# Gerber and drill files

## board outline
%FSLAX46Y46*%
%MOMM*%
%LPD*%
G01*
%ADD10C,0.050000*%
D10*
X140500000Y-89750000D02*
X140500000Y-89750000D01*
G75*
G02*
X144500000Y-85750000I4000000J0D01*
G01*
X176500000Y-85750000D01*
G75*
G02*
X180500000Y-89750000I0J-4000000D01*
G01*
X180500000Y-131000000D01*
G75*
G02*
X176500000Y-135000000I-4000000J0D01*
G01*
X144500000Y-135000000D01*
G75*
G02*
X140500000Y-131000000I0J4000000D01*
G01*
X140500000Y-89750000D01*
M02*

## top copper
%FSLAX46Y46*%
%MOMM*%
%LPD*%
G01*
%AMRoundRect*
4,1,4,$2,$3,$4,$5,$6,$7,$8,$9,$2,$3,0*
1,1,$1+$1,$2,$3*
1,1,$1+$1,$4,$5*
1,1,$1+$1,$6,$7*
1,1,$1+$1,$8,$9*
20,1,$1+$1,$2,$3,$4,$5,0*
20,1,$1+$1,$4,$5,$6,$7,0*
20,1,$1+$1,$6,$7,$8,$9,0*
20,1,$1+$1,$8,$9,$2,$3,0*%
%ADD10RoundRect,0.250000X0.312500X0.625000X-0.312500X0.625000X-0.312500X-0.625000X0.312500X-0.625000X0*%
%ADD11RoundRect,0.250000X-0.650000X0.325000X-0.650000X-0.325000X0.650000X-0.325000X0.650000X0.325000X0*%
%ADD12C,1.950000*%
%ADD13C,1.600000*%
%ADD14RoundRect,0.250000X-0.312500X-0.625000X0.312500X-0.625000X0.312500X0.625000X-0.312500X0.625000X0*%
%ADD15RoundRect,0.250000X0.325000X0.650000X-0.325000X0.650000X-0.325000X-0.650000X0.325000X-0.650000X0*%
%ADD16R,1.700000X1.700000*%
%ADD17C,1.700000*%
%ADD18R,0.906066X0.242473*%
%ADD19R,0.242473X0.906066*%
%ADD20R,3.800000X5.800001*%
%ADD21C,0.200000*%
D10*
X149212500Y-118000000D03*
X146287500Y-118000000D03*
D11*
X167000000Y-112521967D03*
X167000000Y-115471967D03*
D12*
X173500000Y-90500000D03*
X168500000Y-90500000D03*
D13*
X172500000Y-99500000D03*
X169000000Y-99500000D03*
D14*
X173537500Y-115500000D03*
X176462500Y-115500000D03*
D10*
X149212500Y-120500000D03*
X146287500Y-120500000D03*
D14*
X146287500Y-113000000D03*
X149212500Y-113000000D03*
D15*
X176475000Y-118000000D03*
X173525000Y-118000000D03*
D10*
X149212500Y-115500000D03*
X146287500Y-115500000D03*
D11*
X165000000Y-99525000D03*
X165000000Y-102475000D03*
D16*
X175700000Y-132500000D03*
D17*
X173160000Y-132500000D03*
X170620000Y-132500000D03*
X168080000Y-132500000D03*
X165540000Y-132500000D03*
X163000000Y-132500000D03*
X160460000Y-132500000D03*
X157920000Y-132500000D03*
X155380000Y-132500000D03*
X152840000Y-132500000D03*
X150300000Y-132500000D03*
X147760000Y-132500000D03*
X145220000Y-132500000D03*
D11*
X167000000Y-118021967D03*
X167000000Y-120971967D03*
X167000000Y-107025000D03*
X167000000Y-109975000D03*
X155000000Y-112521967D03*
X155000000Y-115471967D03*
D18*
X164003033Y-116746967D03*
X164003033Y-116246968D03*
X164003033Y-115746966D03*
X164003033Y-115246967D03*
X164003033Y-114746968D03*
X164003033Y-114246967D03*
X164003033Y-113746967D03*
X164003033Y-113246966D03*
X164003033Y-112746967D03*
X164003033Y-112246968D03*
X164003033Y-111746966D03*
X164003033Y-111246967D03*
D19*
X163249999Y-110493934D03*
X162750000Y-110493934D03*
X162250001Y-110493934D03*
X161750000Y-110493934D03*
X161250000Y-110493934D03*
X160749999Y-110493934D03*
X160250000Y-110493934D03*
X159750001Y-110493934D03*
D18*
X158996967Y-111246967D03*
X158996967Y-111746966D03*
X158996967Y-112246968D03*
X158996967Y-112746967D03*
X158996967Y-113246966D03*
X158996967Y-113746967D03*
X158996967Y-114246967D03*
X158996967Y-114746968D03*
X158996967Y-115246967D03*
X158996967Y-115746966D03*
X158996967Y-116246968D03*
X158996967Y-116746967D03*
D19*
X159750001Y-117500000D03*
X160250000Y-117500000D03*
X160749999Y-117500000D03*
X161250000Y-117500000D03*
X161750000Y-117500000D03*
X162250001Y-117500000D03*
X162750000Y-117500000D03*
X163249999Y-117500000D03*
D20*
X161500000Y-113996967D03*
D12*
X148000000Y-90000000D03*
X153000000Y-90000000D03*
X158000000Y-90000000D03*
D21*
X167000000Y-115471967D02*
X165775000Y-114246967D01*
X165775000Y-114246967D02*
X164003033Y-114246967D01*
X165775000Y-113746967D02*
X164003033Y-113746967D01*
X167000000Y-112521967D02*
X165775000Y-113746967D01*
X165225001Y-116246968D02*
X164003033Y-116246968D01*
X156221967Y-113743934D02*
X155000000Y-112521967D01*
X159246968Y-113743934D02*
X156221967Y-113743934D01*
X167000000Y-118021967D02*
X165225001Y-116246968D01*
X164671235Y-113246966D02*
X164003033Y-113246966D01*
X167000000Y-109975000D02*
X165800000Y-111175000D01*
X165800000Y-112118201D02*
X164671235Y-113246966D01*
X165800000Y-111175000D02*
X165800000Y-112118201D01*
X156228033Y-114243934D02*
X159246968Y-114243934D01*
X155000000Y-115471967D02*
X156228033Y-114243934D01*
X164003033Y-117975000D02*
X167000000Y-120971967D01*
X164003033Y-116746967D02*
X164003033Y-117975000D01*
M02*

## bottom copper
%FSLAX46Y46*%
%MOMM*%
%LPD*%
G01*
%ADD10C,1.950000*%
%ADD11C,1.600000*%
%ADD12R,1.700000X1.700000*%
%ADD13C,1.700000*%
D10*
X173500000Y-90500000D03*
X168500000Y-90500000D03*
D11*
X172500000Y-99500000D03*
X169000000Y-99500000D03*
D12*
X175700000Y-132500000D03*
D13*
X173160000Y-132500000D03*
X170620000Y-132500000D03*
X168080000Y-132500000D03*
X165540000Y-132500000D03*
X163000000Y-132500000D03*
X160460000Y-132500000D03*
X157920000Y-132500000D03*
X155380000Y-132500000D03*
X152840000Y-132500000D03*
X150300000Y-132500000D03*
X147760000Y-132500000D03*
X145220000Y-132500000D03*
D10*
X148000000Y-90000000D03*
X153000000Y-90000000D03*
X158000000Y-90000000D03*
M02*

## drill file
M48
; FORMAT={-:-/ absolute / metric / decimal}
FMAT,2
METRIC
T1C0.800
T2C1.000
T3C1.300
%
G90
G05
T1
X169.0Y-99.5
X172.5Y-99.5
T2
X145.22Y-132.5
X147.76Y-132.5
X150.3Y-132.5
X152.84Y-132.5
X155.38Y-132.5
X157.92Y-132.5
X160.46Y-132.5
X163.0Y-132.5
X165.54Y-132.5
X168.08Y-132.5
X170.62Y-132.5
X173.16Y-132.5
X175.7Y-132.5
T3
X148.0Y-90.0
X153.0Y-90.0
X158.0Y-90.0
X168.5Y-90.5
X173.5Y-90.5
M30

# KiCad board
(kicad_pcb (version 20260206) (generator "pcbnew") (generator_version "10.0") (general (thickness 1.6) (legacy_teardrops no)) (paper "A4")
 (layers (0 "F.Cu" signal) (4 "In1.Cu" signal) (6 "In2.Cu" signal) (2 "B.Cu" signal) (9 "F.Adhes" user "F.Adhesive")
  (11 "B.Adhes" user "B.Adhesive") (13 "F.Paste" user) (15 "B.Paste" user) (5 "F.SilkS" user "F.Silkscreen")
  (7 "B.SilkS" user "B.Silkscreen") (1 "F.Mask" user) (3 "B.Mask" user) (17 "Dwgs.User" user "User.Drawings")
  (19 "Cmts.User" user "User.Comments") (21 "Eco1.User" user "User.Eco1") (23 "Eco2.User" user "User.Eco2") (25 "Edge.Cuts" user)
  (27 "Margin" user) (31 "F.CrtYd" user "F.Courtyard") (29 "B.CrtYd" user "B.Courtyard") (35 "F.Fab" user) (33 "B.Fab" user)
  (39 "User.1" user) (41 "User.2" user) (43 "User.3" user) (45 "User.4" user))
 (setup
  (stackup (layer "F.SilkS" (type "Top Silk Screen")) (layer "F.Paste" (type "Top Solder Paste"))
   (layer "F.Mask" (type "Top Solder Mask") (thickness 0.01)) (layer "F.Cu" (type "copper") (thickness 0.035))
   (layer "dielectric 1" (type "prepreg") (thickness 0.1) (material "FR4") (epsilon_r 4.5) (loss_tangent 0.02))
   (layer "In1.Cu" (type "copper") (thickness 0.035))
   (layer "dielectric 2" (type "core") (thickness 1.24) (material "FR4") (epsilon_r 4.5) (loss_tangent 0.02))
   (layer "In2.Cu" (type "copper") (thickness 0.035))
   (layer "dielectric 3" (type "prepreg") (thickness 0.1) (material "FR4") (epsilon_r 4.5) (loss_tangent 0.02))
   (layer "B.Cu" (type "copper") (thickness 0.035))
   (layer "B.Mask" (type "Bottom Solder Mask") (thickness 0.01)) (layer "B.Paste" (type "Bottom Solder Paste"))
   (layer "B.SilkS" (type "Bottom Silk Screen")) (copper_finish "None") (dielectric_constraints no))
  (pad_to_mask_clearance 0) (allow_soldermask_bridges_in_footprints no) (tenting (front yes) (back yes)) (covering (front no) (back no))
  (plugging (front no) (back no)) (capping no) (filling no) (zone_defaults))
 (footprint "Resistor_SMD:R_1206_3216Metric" (layer "F.Cu") (at 147.75 118 180)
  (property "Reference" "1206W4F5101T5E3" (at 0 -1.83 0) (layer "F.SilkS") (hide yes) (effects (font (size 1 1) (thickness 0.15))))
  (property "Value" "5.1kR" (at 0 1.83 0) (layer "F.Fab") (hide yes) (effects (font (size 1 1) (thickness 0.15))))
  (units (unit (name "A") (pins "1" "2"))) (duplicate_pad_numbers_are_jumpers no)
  (pad "1" smd roundrect (at -1.4625 0 180) (size 1.125 1.75) (layers "F.Cu" "F.Mask" "F.Paste") (roundrect_rratio 0.222222)
   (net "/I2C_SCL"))
  (pad "2" smd roundrect (at 1.4625 0 180) (size 1.125 1.75) (layers "F.Cu" "F.Mask" "F.Paste") (roundrect_rratio 0.222222) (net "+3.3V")))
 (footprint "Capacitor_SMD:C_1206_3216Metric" (layer "F.Cu") (at 167 113.996967 -90)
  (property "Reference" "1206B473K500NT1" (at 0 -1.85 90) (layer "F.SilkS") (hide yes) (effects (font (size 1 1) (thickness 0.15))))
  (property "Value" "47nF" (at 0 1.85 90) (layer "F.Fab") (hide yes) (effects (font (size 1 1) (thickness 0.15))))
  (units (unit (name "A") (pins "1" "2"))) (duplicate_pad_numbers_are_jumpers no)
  (pad "1" smd roundrect (at -1.475 0 270) (size 1.15 1.8) (layers "F.Cu" "F.Mask" "F.Paste") (roundrect_rratio 0.217391) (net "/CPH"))
  (pad "2" smd roundrect (at 1.475 0 270) (size 1.15 1.8) (layers "F.Cu" "F.Mask" "F.Paste") (roundrect_rratio 0.217391) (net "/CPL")))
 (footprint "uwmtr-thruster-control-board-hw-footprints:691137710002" (layer "F.Cu") (at 171 90.5 180)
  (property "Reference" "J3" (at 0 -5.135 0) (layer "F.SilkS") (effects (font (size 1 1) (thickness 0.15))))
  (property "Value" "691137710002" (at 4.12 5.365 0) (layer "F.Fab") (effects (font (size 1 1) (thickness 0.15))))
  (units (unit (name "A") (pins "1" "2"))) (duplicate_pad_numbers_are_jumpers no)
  (pad "1" thru_hole circle (at -2.5 0 180) (size 1.95 1.95) (drill 1.3) (layers "*.Cu" "*.Mask") (remove_unused_layers no) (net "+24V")
   (solder_mask_margin 0.102))
  (pad "2" thru_hole circle (at 2.5 0 180) (size 1.95 1.95) (drill 1.3) (layers "*.Cu" "*.Mask") (remove_unused_layers no) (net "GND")
   (solder_mask_margin 0.102)))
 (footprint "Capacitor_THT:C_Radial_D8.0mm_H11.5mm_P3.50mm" (layer "F.Cu") (at 172.5 99.5 180)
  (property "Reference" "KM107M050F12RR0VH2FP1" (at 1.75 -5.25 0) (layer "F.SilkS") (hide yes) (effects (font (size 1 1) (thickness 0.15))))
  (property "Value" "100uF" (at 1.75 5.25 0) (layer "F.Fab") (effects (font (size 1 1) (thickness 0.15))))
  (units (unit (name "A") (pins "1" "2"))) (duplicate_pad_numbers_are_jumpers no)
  (pad "1" thru_hole circle (at 0 0 180) (size 1.6 1.6) (drill 0.8) (layers "*.Cu" "*.Mask") (remove_unused_layers no) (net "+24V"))
  (pad "2" thru_hole circle (at 3.5 0 180) (size 1.6 1.6) (drill 0.8) (layers "*.Cu" "*.Mask") (remove_unused_layers no) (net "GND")))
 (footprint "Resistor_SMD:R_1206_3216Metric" (layer "F.Cu") (at 175 115.5)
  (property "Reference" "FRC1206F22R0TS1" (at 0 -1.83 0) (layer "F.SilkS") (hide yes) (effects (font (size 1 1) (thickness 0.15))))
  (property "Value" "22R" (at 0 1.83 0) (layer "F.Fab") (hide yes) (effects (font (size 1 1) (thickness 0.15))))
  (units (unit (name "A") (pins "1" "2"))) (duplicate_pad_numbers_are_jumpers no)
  (pad "1" smd roundrect (at -1.4625 0) (size 1.125 1.75) (layers "F.Cu" "F.Mask" "F.Paste") (roundrect_rratio 0.222222) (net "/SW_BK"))
  (pad "2" smd roundrect (at 1.4625 0) (size 1.125 1.75) (layers "F.Cu" "F.Mask" "F.Paste") (roundrect_rratio 0.222222) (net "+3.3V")))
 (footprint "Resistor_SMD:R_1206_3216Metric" (layer "F.Cu") (at 147.75 120.5 180)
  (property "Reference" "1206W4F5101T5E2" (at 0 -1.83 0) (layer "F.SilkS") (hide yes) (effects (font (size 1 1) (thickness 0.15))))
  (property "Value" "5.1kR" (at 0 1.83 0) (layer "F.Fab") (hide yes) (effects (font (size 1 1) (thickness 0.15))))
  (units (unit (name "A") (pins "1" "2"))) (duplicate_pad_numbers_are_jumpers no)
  (pad "1" smd roundrect (at -1.4625 0 180) (size 1.125 1.75) (layers "F.Cu" "F.Mask" "F.Paste") (roundrect_rratio 0.222222)
   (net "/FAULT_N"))
  (pad "2" smd roundrect (at 1.4625 0 180) (size 1.125 1.75) (layers "F.Cu" "F.Mask" "F.Paste") (roundrect_rratio 0.222222) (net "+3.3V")))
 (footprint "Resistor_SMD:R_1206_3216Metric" (layer "F.Cu") (at 147.75 113)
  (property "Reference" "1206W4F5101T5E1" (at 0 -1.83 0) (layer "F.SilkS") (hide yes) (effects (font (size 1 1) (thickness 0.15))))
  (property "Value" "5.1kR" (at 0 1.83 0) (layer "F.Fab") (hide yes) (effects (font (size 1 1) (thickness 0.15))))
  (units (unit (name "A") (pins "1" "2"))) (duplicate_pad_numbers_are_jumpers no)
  (pad "1" smd roundrect (at -1.4625 0) (size 1.125 1.75) (layers "F.Cu" "F.Mask" "F.Paste") (roundrect_rratio 0.222222) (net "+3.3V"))
  (pad "2" smd roundrect (at 1.4625 0) (size 1.125 1.75) (layers "F.Cu" "F.Mask" "F.Paste") (roundrect_rratio 0.222222) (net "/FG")))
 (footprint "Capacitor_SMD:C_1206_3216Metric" (layer "F.Cu") (at 175 118 180)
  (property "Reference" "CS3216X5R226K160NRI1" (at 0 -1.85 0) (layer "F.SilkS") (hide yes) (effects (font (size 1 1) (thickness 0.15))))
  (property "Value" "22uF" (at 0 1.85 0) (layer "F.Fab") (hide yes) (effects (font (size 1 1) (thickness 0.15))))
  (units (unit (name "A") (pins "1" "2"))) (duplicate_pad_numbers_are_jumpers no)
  (pad "1" smd roundrect (at -1.475 0 180) (size 1.15 1.8) (layers "F.Cu" "F.Mask" "F.Paste") (roundrect_rratio 0.217391) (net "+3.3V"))
  (pad "2" smd roundrect (at 1.475 0 180) (size 1.15 1.8) (layers "F.Cu" "F.Mask" "F.Paste") (roundrect_rratio 0.217391) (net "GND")))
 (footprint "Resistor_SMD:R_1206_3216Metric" (layer "F.Cu") (at 147.75 115.5 180)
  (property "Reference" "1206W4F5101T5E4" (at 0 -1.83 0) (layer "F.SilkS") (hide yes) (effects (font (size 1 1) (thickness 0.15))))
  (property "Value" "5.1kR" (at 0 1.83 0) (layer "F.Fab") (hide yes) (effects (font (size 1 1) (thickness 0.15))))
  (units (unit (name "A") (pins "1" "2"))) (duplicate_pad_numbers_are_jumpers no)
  (pad "1" smd roundrect (at -1.4625 0 180) (size 1.125 1.75) (layers "F.Cu" "F.Mask" "F.Paste") (roundrect_rratio 0.222222)
   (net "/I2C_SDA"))
  (pad "2" smd roundrect (at 1.4625 0 180) (size 1.125 1.75) (layers "F.Cu" "F.Mask" "F.Paste") (roundrect_rratio 0.222222) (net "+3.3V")))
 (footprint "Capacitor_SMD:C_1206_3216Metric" (layer "F.Cu") (at 165 101 -90)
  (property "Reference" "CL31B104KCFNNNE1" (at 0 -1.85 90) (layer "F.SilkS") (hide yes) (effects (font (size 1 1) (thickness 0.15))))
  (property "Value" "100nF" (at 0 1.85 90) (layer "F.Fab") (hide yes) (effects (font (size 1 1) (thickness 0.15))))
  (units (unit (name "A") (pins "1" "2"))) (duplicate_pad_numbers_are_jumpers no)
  (pad "1" smd roundrect (at -1.475 0 270) (size 1.15 1.8) (layers "F.Cu" "F.Mask" "F.Paste") (roundrect_rratio 0.217391) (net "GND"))
  (pad "2" smd roundrect (at 1.475 0 270) (size 1.15 1.8) (layers "F.Cu" "F.Mask" "F.Paste") (roundrect_rratio 0.217391) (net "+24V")))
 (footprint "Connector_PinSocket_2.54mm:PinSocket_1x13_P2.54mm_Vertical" (layer "F.Cu") (at 175.7 132.5 -90)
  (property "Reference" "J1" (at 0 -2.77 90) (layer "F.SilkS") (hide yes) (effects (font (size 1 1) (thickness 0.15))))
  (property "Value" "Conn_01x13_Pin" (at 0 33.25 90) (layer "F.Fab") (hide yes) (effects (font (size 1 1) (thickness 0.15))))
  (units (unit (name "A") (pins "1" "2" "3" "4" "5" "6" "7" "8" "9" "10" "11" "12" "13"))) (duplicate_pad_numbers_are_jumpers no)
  (pad "1" thru_hole rect (at 0 0 270) (size 1.7 1.7) (drill 1) (layers "*.Cu" "*.Mask") (remove_unused_layers no) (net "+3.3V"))
  (pad "2" thru_hole circle (at 0 2.54 270) (size 1.7 1.7) (drill 1) (layers "*.Cu" "*.Mask") (remove_unused_layers no) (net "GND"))
  (pad "3" thru_hole circle (at 0 5.08 270) (size 1.7 1.7) (drill 1) (layers "*.Cu" "*.Mask") (remove_unused_layers no) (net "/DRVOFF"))
  (pad "4" thru_hole circle (at 0 7.62 270) (size 1.7 1.7) (drill 1) (layers "*.Cu" "*.Mask") (remove_unused_layers no) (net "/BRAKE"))
  (pad "5" thru_hole circle (at 0 10.16 270) (size 1.7 1.7) (drill 1) (layers "*.Cu" "*.Mask") (remove_unused_layers no) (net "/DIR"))
  (pad "6" thru_hole circle (at 0 12.7 270) (size 1.7 1.7) (drill 1) (layers "*.Cu" "*.Mask") (remove_unused_layers no) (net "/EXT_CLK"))
  (pad "7" thru_hole circle (at 0 15.24 270) (size 1.7 1.7) (drill 1) (layers "*.Cu" "*.Mask") (remove_unused_layers no) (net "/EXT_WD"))
  (pad "8" thru_hole circle (at 0 17.78 270) (size 1.7 1.7) (drill 1) (layers "*.Cu" "*.Mask") (remove_unused_layers no) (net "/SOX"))
  (pad "9" thru_hole circle (at 0 20.32 270) (size 1.7 1.7) (drill 1) (layers "*.Cu" "*.Mask") (remove_unused_layers no) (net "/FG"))
  (pad "10" thru_hole circle (at 0 22.86 270) (size 1.7 1.7) (drill 1) (layers "*.Cu" "*.Mask") (remove_unused_layers no) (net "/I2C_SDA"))
  (pad "11" thru_hole circle (at 0 25.4 270) (size 1.7 1.7) (drill 1) (layers "*.Cu" "*.Mask") (remove_unused_layers no) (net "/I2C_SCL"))
  (pad "12" thru_hole circle (at 0 27.94 270) (size 1.7 1.7) (drill 1) (layers "*.Cu" "*.Mask") (remove_unused_layers no) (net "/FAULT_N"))
  (pad "13" thru_hole circle (at 0 30.48 270) (size 1.7 1.7) (drill 1) (layers "*.Cu" "*.Mask") (remove_unused_layers no)
   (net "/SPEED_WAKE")))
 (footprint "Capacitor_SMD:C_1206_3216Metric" (layer "F.Cu") (at 167 119.496967 -90)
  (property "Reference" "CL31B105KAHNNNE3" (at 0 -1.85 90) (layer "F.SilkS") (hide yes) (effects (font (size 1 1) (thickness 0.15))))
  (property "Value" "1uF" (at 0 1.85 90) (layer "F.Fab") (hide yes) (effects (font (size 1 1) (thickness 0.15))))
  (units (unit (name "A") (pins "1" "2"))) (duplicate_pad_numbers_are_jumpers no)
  (pad "1" smd roundrect (at -1.475 0 270) (size 1.15 1.8) (layers "F.Cu" "F.Mask" "F.Paste") (roundrect_rratio 0.217391) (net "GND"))
  (pad "2" smd roundrect (at 1.475 0 270) (size 1.15 1.8) (layers "F.Cu" "F.Mask" "F.Paste") (roundrect_rratio 0.217391) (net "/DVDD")))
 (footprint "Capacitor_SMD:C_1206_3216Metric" (layer "F.Cu") (at 167 108.5 -90)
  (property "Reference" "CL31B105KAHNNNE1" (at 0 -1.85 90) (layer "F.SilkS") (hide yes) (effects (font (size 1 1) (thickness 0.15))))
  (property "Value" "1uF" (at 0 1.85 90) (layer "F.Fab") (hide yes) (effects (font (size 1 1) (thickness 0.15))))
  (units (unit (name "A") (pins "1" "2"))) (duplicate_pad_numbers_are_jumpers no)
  (pad "1" smd roundrect (at -1.475 0 270) (size 1.15 1.8) (layers "F.Cu" "F.Mask" "F.Paste") (roundrect_rratio 0.217391) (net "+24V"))
  (pad "2" smd roundrect (at 1.475 0 270) (size 1.15 1.8) (layers "F.Cu" "F.Mask" "F.Paste") (roundrect_rratio 0.217391) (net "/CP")))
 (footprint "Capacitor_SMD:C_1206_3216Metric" (layer "F.Cu") (at 155 113.996967 -90)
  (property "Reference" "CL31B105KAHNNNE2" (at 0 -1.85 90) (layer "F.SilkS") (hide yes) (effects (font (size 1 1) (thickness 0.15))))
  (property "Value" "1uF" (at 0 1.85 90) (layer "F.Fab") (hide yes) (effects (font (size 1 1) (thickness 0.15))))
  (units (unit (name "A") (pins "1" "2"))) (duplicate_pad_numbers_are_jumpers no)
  (pad "1" smd roundrect (at -1.475 0 270) (size 1.15 1.8) (layers "F.Cu" "F.Mask" "F.Paste") (roundrect_rratio 0.217391) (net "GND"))
  (pad "2" smd roundrect (at 1.475 0 270) (size 1.15 1.8) (layers "F.Cu" "F.Mask" "F.Paste") (roundrect_rratio 0.217391) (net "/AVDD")))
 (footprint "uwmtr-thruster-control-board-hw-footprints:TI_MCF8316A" (layer "F.Cu") (at 161.5 113.996967 180)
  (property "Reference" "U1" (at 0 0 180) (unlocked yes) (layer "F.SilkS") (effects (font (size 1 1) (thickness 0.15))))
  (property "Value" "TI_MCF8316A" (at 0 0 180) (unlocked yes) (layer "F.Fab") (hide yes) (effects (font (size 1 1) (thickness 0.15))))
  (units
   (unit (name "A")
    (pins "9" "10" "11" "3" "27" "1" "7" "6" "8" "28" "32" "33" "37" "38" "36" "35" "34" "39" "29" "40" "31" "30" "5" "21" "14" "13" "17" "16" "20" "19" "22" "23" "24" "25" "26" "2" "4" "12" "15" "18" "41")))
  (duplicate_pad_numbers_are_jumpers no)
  (pad "1" smd rect (at -2.503033 -2.75 270) (size 0.242473 0.906066) (layers "F.Cu" "F.Mask" "F.Paste") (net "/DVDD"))
  (pad "2" smd rect (at -2.503033 -2.250001 270) (size 0.242473 0.906066) (layers "F.Cu" "F.Mask" "F.Paste") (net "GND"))
  (pad "3" smd rect (at -2.503033 -1.749999 270) (size 0.242473 0.906066) (layers "F.Cu" "F.Mask" "F.Paste") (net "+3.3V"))
  (pad "4" smd rect (at -2.503033 -1.25 270) (size 0.242473 0.906066) (layers "F.Cu" "F.Mask" "F.Paste") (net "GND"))
  (pad "5" smd rect (at -2.503033 -0.750001 270) (size 0.242473 0.906066) (layers "F.Cu" "F.Mask" "F.Paste") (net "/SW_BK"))
  (pad "6" smd rect (at -2.503033 -0.25 270) (size 0.242473 0.906066) (layers "F.Cu" "F.Mask" "F.Paste") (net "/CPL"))
  (pad "7" smd rect (at -2.503033 0.25 270) (size 0.242473 0.906066) (layers "F.Cu" "F.Mask" "F.Paste") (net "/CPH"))
  (pad "8" smd rect (at -2.503033 0.750001 270) (size 0.242473 0.906066) (layers "F.Cu" "F.Mask" "F.Paste") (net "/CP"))
  (pad "9" smd rect (at -2.503033 1.25 270) (size 0.242473 0.906066) (layers "F.Cu" "F.Mask" "F.Paste") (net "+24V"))
  (pad "10" smd rect (at -2.503033 1.749999 270) (size 0.242473 0.906066) (layers "F.Cu" "F.Mask" "F.Paste") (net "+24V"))
  (pad "11" smd rect (at -2.503033 2.250001 270) (size 0.242473 0.906066) (layers "F.Cu" "F.Mask" "F.Paste") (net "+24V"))
  (pad "12" smd rect (at -2.503033 2.75 270) (size 0.242473 0.906066) (layers "F.Cu" "F.Mask" "F.Paste") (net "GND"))
  (pad "13" smd rect (at -1.749999 3.503033 180) (size 0.242473 0.906066) (layers "F.Cu" "F.Mask" "F.Paste") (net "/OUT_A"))
  (pad "14" smd rect (at -1.25 3.503033 180) (size 0.242473 0.906066) (layers "F.Cu" "F.Mask" "F.Paste") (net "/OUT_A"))
  (pad "15" smd rect (at -0.750001 3.503033 180) (size 0.242473 0.906066) (layers "F.Cu" "F.Mask" "F.Paste") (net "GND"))
  (pad "16" smd rect (at -0.25 3.503033 180) (size 0.242473 0.906066) (layers "F.Cu" "F.Mask" "F.Paste") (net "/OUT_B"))
  (pad "17" smd rect (at 0.25 3.503033 180) (size 0.242473 0.906066) (layers "F.Cu" "F.Mask" "F.Paste") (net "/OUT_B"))
  (pad "18" smd rect (at 0.750001 3.503033 180) (size 0.242473 0.906066) (layers "F.Cu" "F.Mask" "F.Paste") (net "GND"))
  (pad "19" smd rect (at 1.25 3.503033 180) (size 0.242473 0.906066) (layers "F.Cu" "F.Mask" "F.Paste") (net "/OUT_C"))
  (pad "20" smd rect (at 1.749999 3.503033 180) (size 0.242473 0.906066) (layers "F.Cu" "F.Mask" "F.Paste") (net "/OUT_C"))
  (pad "21" smd rect (at 2.503033 2.75 270) (size 0.242473 0.906066) (layers "F.Cu" "F.Mask" "F.Paste") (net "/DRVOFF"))
  (pad "22" smd rect (at 2.503033 2.250001 270) (size 0.242473 0.906066) (layers "F.Cu" "F.Mask" "F.Paste")
   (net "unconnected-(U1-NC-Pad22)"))
  (pad "23" smd rect (at 2.503033 1.749999 270) (size 0.242473 0.906066) (layers "F.Cu" "F.Mask" "F.Paste")
   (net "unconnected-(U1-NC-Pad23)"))
  (pad "24" smd rect (at 2.503033 1.25 270) (size 0.242473 0.906066) (layers "F.Cu" "F.Mask" "F.Paste") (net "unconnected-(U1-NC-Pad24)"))
  (pad "25" smd rect (at 2.503033 0.750001 270) (size 0.242473 0.906066) (layers "F.Cu" "F.Mask" "F.Paste")
   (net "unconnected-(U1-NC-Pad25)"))
  (pad "26" smd rect (at 2.503033 0.25 270) (size 0.242473 0.906066) (layers "F.Cu" "F.Mask" "F.Paste") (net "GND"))
  (pad "27" smd rect (at 2.503033 -0.25 270) (size 0.242473 0.906066) (layers "F.Cu" "F.Mask" "F.Paste") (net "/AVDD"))
  (pad "28" smd rect (at 2.503033 -0.750001 270) (size 0.242473 0.906066) (layers "F.Cu" "F.Mask" "F.Paste") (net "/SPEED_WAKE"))
  (pad "29" smd rect (at 2.503033 -1.25 270) (size 0.242473 0.906066) (layers "F.Cu" "F.Mask" "F.Paste") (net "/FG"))
  (pad "30" smd rect (at 2.503033 -1.749999 270) (size 0.242473 0.906066) (layers "F.Cu" "F.Mask" "F.Paste") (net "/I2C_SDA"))
  (pad "31" smd rect (at 2.503033 -2.250001 270) (size 0.242473 0.906066) (layers "F.Cu" "F.Mask" "F.Paste") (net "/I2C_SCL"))
  (pad "32" smd rect (at 2.503033 -2.75 270) (size 0.242473 0.906066) (layers "F.Cu" "F.Mask" "F.Paste") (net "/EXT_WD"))
  (pad "33" smd rect (at 1.749999 -3.503033 180) (size 0.242473 0.906066) (layers "F.Cu" "F.Mask" "F.Paste") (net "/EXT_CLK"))
  (pad "34" smd rect (at 1.25 -3.503033 180) (size 0.242473 0.906066) (layers "F.Cu" "F.Mask" "F.Paste") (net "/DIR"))
  (pad "35" smd rect (at 0.750001 -3.503033 180) (size 0.242473 0.906066) (layers "F.Cu" "F.Mask" "F.Paste") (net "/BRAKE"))
  (pad "36" smd rect (at 0.25 -3.503033 180) (size 0.242473 0.906066) (layers "F.Cu" "F.Mask" "F.Paste") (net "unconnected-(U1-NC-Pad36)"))
  (pad "37" smd rect (at -0.25 -3.503033 180) (size 0.242473 0.906066) (layers "F.Cu" "F.Mask" "F.Paste") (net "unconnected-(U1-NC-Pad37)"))
  (pad "38" smd rect (at -0.750001 -3.503033 180) (size 0.242473 0.906066) (layers "F.Cu" "F.Mask" "F.Paste") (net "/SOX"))
  (pad "39" smd rect (at -1.25 -3.503033 180) (size 0.242473 0.906066) (layers "F.Cu" "F.Mask" "F.Paste") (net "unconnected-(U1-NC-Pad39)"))
  (pad "40" smd rect (at -1.749999 -3.503033 180) (size 0.242473 0.906066) (layers "F.Cu" "F.Mask" "F.Paste") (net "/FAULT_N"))
  (pad "41" smd rect (at 0 0 180) (size 3.8 5.800001) (layers "F.Cu" "F.Mask") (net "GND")))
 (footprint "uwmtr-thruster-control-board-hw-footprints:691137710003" (layer "F.Cu") (at 153 90)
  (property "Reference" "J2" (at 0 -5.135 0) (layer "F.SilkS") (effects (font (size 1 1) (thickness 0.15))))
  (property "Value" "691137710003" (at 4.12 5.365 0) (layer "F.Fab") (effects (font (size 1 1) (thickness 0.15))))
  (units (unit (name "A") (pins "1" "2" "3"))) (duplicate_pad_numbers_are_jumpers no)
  (pad "1" thru_hole circle (at -5 0) (size 1.95 1.95) (drill 1.3) (layers "*.Cu" "*.Mask") (remove_unused_layers no) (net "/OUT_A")
   (solder_mask_margin 0.102))
  (pad "2" thru_hole circle (at 0 0) (size 1.95 1.95) (drill 1.3) (layers "*.Cu" "*.Mask") (remove_unused_layers no) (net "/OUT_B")
   (solder_mask_margin 0.102))
  (pad "3" thru_hole circle (at 5 0) (size 1.95 1.95) (drill 1.3) (layers "*.Cu" "*.Mask") (remove_unused_layers no) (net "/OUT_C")
   (solder_mask_margin 0.102)))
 (gr_rect (start 140.5 85.75) (end 180.5 135) (radius 4) (stroke (width 0.05) (type solid)) (fill no) (layer "Edge.Cuts"))
 (segment (start 167 115.471967) (end 165.775 114.246967) (width 0.2) (layer "F.Cu") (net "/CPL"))
 (segment (start 165.775 114.246967) (end 164.003033 114.246967) (width 0.2) (layer "F.Cu") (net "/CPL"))
 (segment (start 165.775 113.746967) (end 164.003033 113.746967) (width 0.2) (layer "F.Cu") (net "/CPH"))
 (segment (start 167 112.521967) (end 165.775 113.746967) (width 0.2) (layer "F.Cu") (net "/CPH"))
 (segment (start 165.225001 116.246968) (end 164.003033 116.246968) (width 0.2) (layer "F.Cu") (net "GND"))
 (segment (start 156.221967 113.743934) (end 155 112.521967) (width 0.2) (layer "F.Cu") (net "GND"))
 (segment (start 159.246968 113.743934) (end 156.221967 113.743934) (width 0.2) (layer "F.Cu") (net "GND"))
 (segment (start 167 118.021967) (end 165.225001 116.246968) (width 0.2) (layer "F.Cu") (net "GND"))
 (segment (start 164.671235 113.246966) (end 164.003033 113.246966) (width 0.2) (layer "F.Cu") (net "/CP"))
 (segment (start 167 109.975) (end 165.8 111.175) (width 0.2) (layer "F.Cu") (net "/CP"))
 (segment (start 165.8 112.118201) (end 164.671235 113.246966) (width 0.2) (layer "F.Cu") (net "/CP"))
 (segment (start 165.8 111.175) (end 165.8 112.118201) (width 0.2) (layer "F.Cu") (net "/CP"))
 (segment (start 156.228033 114.243934) (end 159.246968 114.243934) (width 0.2) (layer "F.Cu") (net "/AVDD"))
 (segment (start 155 115.471967) (end 156.228033 114.243934) (width 0.2) (layer "F.Cu") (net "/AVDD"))
 (segment (start 164.003033 117.975) (end 167 120.971967) (width 0.2) (layer "F.Cu") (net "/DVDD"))
 (segment (start 164.003033 116.746967) (end 164.003033 117.975) (width 0.2) (layer "F.Cu") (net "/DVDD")))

